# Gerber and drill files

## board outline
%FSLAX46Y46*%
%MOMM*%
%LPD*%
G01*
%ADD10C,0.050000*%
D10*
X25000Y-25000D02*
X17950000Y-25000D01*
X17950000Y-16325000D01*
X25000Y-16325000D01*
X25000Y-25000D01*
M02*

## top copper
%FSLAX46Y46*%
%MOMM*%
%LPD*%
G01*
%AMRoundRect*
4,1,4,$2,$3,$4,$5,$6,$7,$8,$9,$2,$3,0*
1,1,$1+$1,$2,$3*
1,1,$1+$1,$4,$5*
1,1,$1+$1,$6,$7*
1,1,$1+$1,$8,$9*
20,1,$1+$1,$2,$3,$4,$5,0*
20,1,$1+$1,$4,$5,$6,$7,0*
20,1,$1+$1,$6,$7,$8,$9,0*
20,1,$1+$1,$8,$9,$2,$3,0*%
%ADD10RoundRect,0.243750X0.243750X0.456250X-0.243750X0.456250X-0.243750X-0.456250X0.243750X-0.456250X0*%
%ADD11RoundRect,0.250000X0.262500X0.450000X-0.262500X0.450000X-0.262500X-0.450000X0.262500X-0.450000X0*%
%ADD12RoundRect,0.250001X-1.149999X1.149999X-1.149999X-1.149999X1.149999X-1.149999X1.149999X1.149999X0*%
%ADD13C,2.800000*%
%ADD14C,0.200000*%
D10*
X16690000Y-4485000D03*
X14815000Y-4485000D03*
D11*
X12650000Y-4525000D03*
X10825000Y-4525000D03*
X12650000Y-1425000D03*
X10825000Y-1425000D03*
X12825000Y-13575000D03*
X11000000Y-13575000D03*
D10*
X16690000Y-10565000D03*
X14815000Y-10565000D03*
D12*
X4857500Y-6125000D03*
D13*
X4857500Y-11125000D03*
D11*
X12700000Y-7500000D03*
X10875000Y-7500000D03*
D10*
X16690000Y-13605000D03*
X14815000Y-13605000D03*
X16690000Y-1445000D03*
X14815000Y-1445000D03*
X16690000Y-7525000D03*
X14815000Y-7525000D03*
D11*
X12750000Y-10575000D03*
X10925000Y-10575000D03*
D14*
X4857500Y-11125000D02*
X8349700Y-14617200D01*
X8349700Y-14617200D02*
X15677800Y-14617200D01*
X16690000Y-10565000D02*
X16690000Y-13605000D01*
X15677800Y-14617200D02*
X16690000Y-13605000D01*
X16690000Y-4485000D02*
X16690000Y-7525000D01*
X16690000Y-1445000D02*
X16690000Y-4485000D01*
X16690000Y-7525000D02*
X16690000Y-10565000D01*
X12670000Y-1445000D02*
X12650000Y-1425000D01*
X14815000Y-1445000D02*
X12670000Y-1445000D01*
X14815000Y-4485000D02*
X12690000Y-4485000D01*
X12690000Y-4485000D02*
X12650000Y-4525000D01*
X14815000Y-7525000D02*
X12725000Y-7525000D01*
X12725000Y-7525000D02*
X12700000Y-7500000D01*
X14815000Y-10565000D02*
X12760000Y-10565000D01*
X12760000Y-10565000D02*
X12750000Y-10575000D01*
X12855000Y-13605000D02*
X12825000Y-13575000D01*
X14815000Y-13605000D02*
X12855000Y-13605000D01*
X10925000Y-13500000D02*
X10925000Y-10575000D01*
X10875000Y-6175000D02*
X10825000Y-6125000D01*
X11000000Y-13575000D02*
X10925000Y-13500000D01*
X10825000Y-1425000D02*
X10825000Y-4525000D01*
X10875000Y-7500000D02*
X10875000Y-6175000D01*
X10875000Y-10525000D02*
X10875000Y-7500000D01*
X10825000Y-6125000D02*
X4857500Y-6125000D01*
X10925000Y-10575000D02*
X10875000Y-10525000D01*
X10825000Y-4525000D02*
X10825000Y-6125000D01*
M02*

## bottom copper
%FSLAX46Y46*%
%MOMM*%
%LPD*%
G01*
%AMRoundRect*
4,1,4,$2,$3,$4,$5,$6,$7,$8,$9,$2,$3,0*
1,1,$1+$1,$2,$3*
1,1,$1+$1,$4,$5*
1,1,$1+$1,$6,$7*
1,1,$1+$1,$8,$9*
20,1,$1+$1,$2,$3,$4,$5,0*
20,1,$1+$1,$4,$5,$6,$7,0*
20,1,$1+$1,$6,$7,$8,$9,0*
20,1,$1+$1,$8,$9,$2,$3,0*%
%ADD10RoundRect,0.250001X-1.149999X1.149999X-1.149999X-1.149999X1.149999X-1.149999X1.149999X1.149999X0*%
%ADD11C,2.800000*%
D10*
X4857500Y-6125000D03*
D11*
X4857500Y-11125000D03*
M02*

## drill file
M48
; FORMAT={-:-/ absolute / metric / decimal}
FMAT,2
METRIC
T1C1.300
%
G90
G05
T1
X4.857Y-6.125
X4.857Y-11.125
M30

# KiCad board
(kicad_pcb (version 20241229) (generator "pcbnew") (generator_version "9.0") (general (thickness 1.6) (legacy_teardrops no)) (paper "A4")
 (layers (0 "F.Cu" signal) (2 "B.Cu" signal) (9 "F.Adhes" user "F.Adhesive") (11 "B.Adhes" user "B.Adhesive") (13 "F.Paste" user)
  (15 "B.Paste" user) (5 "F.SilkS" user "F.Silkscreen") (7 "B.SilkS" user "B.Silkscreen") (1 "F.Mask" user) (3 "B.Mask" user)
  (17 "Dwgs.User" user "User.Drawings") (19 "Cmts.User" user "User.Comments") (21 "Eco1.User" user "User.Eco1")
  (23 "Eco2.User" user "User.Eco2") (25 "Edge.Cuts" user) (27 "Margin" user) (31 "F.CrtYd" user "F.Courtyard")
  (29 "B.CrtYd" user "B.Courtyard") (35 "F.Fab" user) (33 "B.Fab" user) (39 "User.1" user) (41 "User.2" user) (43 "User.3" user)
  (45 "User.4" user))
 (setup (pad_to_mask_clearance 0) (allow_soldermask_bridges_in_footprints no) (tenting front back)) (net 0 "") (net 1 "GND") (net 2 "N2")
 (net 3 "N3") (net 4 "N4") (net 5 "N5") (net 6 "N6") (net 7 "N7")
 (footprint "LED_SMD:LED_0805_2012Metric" (layer "F.Cu") (at 15.7525 4.485 180)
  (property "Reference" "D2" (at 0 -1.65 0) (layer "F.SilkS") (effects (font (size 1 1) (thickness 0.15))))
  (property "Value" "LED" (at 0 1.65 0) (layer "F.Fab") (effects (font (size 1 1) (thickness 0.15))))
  (pad "1" smd roundrect (at -0.9375 0 180) (size 0.975 1.4) (layers "F.Cu" "F.Mask" "F.Paste") (roundrect_rratio 0.25) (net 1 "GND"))
  (pad "2" smd roundrect (at 0.9375 0 180) (size 0.975 1.4) (layers "F.Cu" "F.Mask" "F.Paste") (roundrect_rratio 0.25) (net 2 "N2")))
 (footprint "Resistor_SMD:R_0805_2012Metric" (layer "F.Cu") (at 11.7375 4.525 180)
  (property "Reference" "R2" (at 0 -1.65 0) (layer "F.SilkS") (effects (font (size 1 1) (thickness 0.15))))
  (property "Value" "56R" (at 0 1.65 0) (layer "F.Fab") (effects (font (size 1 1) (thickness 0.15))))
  (pad "1" smd roundrect (at -0.9125 0 180) (size 1.025 1.4) (layers "F.Cu" "F.Mask" "F.Paste") (roundrect_rratio 0.243902) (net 2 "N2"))
  (pad "2" smd roundrect (at 0.9125 0 180) (size 1.025 1.4) (layers "F.Cu" "F.Mask" "F.Paste") (roundrect_rratio 0.243902) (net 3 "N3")))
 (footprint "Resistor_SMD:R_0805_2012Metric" (layer "F.Cu") (at 11.7375 1.425 180)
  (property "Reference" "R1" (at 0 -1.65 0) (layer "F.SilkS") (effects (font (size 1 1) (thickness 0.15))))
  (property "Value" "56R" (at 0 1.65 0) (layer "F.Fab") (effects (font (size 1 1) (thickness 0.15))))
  (pad "1" smd roundrect (at -0.9125 0 180) (size 1.025 1.4) (layers "F.Cu" "F.Mask" "F.Paste") (roundrect_rratio 0.243902) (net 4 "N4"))
  (pad "2" smd roundrect (at 0.9125 0 180) (size 1.025 1.4) (layers "F.Cu" "F.Mask" "F.Paste") (roundrect_rratio 0.243902) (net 3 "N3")))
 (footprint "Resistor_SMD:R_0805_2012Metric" (layer "F.Cu") (at 11.9125 13.575 180)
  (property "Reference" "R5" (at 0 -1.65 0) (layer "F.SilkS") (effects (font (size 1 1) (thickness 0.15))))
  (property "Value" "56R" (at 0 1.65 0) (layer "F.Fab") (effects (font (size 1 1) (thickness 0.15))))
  (pad "1" smd roundrect (at -0.9125 0 180) (size 1.025 1.4) (layers "F.Cu" "F.Mask" "F.Paste") (roundrect_rratio 0.243902) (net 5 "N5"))
  (pad "2" smd roundrect (at 0.9125 0 180) (size 1.025 1.4) (layers "F.Cu" "F.Mask" "F.Paste") (roundrect_rratio 0.243902) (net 3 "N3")))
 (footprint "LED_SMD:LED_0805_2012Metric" (layer "F.Cu") (at 15.7525 10.565 180)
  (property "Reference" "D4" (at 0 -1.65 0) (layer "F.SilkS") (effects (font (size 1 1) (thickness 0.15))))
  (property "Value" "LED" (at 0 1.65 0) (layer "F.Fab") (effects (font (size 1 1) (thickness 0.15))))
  (pad "1" smd roundrect (at -0.9375 0 180) (size 0.975 1.4) (layers "F.Cu" "F.Mask" "F.Paste") (roundrect_rratio 0.25) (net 1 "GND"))
  (pad "2" smd roundrect (at 0.9375 0 180) (size 0.975 1.4) (layers "F.Cu" "F.Mask" "F.Paste") (roundrect_rratio 0.25) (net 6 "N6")))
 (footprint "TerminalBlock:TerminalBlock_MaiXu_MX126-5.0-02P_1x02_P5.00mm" (layer "F.Cu") (at 4.8575 6.125 -90)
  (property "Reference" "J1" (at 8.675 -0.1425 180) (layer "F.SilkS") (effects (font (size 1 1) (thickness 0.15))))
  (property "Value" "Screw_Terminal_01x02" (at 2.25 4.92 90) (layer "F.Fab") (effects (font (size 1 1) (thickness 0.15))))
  (pad "1" thru_hole roundrect (at 0 0 270) (size 2.8 2.8) (drill 1.3) (layers "*.Cu" "*.Mask") (remove_unused_layers no)
   (roundrect_rratio 0.089286) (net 3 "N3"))
  (pad "2" thru_hole circle (at 5 0 270) (size 2.8 2.8) (drill 1.3) (layers "*.Cu" "*.Mask") (remove_unused_layers no) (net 1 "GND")))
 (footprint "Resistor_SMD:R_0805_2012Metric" (layer "F.Cu") (at 11.7875 7.5 180)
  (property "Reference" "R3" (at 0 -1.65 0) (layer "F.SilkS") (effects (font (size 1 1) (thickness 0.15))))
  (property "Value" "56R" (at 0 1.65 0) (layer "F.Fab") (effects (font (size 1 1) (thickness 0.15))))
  (pad "1" smd roundrect (at -0.9125 0 180) (size 1.025 1.4) (layers "F.Cu" "F.Mask" "F.Paste") (roundrect_rratio 0.243902) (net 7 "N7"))
  (pad "2" smd roundrect (at 0.9125 0 180) (size 1.025 1.4) (layers "F.Cu" "F.Mask" "F.Paste") (roundrect_rratio 0.243902) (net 3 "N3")))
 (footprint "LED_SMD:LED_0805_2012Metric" (layer "F.Cu") (at 15.7525 13.605 180)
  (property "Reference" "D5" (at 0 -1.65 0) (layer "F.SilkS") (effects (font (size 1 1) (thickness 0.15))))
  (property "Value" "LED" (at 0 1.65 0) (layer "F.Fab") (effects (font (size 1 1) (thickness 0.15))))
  (pad "1" smd roundrect (at -0.9375 0 180) (size 0.975 1.4) (layers "F.Cu" "F.Mask" "F.Paste") (roundrect_rratio 0.25) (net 1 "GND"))
  (pad "2" smd roundrect (at 0.9375 0 180) (size 0.975 1.4) (layers "F.Cu" "F.Mask" "F.Paste") (roundrect_rratio 0.25) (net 5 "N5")))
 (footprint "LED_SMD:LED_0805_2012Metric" (layer "F.Cu") (at 15.7525 1.445 180)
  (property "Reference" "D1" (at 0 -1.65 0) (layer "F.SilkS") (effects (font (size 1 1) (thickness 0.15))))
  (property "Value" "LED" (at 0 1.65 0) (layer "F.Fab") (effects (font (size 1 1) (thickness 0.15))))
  (pad "1" smd roundrect (at -0.9375 0 180) (size 0.975 1.4) (layers "F.Cu" "F.Mask" "F.Paste") (roundrect_rratio 0.25) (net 1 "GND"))
  (pad "2" smd roundrect (at 0.9375 0 180) (size 0.975 1.4) (layers "F.Cu" "F.Mask" "F.Paste") (roundrect_rratio 0.25) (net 4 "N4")))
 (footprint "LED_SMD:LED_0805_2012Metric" (layer "F.Cu") (at 15.7525 7.525 180)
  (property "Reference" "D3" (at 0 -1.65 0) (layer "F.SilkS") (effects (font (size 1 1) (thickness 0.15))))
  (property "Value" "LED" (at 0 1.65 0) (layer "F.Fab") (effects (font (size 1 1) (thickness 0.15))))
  (pad "1" smd roundrect (at -0.9375 0 180) (size 0.975 1.4) (layers "F.Cu" "F.Mask" "F.Paste") (roundrect_rratio 0.25) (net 1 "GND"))
  (pad "2" smd roundrect (at 0.9375 0 180) (size 0.975 1.4) (layers "F.Cu" "F.Mask" "F.Paste") (roundrect_rratio 0.25) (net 7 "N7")))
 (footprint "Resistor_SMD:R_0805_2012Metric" (layer "F.Cu") (at 11.8375 10.575 180)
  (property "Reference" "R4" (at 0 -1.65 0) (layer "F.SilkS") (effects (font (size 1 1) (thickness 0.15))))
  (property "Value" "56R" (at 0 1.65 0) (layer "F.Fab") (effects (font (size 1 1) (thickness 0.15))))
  (pad "1" smd roundrect (at -0.9125 0 180) (size 1.025 1.4) (layers "F.Cu" "F.Mask" "F.Paste") (roundrect_rratio 0.243902) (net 6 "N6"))
  (pad "2" smd roundrect (at 0.9125 0 180) (size 1.025 1.4) (layers "F.Cu" "F.Mask" "F.Paste") (roundrect_rratio 0.243902) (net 3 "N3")))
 (gr_rect (start 0.025 0.025) (end 17.95 16.325) (stroke (width 0.05) (type default)) (fill no) (layer "Edge.Cuts"))
 (segment (start 4.8575 11.125) (end 8.3497 14.6172) (width 0.2) (layer "F.Cu") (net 1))
 (segment (start 8.3497 14.6172) (end 15.6778 14.6172) (width 0.2) (layer "F.Cu") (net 1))
 (segment (start 16.69 10.565) (end 16.69 13.605) (width 0.2) (layer "F.Cu") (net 1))
 (segment (start 15.6778 14.6172) (end 16.69 13.605) (width 0.2) (layer "F.Cu") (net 1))
 (segment (start 16.69 4.485) (end 16.69 7.525) (width 0.2) (layer "F.Cu") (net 1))
 (segment (start 16.69 1.445) (end 16.69 4.485) (width 0.2) (layer "F.Cu") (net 1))
 (segment (start 16.69 7.525) (end 16.69 10.565) (width 0.2) (layer "F.Cu") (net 1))
 (segment (start 12.67 1.445) (end 12.65 1.425) (width 0.2) (layer "F.Cu") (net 4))
 (segment (start 14.815 1.445) (end 12.67 1.445) (width 0.2) (layer "F.Cu") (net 4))
 (segment (start 14.815 4.485) (end 12.69 4.485) (width 0.2) (layer "F.Cu") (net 2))
 (segment (start 12.69 4.485) (end 12.65 4.525) (width 0.2) (layer "F.Cu") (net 2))
 (segment (start 14.815 7.525) (end 12.725 7.525) (width 0.2) (layer "F.Cu") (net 7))
 (segment (start 12.725 7.525) (end 12.7 7.5) (width 0.2) (layer "F.Cu") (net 7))
 (segment (start 14.815 10.565) (end 12.76 10.565) (width 0.2) (layer "F.Cu") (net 6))
 (segment (start 12.76 10.565) (end 12.75 10.575) (width 0.2) (layer "F.Cu") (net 6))
 (segment (start 12.855 13.605) (end 12.825 13.575) (width 0.2) (layer "F.Cu") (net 5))
 (segment (start 14.815 13.605) (end 12.855 13.605) (width 0.2) (layer "F.Cu") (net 5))
 (segment (start 10.925 13.5) (end 10.925 10.575) (width 0.2) (layer "F.Cu") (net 3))
 (segment (start 10.875 6.175) (end 10.825 6.125) (width 0.2) (layer "F.Cu") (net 3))
 (segment (start 11 13.575) (end 10.925 13.5) (width 0.2) (layer "F.Cu") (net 3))
 (segment (start 10.825 1.425) (end 10.825 4.525) (width 0.2) (layer "F.Cu") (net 3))
 (segment (start 10.875 7.5) (end 10.875 6.175) (width 0.2) (layer "F.Cu") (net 3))
 (segment (start 10.875 10.525) (end 10.875 7.5) (width 0.2) (layer "F.Cu") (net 3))
 (segment (start 10.825 6.125) (end 4.8575 6.125) (width 0.2) (layer "F.Cu") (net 3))
 (segment (start 10.925 10.575) (end 10.875 10.525) (width 0.2) (layer "F.Cu") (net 3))
 (segment (start 10.825 4.525) (end 10.825 6.125) (width 0.2) (layer "F.Cu") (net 3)))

